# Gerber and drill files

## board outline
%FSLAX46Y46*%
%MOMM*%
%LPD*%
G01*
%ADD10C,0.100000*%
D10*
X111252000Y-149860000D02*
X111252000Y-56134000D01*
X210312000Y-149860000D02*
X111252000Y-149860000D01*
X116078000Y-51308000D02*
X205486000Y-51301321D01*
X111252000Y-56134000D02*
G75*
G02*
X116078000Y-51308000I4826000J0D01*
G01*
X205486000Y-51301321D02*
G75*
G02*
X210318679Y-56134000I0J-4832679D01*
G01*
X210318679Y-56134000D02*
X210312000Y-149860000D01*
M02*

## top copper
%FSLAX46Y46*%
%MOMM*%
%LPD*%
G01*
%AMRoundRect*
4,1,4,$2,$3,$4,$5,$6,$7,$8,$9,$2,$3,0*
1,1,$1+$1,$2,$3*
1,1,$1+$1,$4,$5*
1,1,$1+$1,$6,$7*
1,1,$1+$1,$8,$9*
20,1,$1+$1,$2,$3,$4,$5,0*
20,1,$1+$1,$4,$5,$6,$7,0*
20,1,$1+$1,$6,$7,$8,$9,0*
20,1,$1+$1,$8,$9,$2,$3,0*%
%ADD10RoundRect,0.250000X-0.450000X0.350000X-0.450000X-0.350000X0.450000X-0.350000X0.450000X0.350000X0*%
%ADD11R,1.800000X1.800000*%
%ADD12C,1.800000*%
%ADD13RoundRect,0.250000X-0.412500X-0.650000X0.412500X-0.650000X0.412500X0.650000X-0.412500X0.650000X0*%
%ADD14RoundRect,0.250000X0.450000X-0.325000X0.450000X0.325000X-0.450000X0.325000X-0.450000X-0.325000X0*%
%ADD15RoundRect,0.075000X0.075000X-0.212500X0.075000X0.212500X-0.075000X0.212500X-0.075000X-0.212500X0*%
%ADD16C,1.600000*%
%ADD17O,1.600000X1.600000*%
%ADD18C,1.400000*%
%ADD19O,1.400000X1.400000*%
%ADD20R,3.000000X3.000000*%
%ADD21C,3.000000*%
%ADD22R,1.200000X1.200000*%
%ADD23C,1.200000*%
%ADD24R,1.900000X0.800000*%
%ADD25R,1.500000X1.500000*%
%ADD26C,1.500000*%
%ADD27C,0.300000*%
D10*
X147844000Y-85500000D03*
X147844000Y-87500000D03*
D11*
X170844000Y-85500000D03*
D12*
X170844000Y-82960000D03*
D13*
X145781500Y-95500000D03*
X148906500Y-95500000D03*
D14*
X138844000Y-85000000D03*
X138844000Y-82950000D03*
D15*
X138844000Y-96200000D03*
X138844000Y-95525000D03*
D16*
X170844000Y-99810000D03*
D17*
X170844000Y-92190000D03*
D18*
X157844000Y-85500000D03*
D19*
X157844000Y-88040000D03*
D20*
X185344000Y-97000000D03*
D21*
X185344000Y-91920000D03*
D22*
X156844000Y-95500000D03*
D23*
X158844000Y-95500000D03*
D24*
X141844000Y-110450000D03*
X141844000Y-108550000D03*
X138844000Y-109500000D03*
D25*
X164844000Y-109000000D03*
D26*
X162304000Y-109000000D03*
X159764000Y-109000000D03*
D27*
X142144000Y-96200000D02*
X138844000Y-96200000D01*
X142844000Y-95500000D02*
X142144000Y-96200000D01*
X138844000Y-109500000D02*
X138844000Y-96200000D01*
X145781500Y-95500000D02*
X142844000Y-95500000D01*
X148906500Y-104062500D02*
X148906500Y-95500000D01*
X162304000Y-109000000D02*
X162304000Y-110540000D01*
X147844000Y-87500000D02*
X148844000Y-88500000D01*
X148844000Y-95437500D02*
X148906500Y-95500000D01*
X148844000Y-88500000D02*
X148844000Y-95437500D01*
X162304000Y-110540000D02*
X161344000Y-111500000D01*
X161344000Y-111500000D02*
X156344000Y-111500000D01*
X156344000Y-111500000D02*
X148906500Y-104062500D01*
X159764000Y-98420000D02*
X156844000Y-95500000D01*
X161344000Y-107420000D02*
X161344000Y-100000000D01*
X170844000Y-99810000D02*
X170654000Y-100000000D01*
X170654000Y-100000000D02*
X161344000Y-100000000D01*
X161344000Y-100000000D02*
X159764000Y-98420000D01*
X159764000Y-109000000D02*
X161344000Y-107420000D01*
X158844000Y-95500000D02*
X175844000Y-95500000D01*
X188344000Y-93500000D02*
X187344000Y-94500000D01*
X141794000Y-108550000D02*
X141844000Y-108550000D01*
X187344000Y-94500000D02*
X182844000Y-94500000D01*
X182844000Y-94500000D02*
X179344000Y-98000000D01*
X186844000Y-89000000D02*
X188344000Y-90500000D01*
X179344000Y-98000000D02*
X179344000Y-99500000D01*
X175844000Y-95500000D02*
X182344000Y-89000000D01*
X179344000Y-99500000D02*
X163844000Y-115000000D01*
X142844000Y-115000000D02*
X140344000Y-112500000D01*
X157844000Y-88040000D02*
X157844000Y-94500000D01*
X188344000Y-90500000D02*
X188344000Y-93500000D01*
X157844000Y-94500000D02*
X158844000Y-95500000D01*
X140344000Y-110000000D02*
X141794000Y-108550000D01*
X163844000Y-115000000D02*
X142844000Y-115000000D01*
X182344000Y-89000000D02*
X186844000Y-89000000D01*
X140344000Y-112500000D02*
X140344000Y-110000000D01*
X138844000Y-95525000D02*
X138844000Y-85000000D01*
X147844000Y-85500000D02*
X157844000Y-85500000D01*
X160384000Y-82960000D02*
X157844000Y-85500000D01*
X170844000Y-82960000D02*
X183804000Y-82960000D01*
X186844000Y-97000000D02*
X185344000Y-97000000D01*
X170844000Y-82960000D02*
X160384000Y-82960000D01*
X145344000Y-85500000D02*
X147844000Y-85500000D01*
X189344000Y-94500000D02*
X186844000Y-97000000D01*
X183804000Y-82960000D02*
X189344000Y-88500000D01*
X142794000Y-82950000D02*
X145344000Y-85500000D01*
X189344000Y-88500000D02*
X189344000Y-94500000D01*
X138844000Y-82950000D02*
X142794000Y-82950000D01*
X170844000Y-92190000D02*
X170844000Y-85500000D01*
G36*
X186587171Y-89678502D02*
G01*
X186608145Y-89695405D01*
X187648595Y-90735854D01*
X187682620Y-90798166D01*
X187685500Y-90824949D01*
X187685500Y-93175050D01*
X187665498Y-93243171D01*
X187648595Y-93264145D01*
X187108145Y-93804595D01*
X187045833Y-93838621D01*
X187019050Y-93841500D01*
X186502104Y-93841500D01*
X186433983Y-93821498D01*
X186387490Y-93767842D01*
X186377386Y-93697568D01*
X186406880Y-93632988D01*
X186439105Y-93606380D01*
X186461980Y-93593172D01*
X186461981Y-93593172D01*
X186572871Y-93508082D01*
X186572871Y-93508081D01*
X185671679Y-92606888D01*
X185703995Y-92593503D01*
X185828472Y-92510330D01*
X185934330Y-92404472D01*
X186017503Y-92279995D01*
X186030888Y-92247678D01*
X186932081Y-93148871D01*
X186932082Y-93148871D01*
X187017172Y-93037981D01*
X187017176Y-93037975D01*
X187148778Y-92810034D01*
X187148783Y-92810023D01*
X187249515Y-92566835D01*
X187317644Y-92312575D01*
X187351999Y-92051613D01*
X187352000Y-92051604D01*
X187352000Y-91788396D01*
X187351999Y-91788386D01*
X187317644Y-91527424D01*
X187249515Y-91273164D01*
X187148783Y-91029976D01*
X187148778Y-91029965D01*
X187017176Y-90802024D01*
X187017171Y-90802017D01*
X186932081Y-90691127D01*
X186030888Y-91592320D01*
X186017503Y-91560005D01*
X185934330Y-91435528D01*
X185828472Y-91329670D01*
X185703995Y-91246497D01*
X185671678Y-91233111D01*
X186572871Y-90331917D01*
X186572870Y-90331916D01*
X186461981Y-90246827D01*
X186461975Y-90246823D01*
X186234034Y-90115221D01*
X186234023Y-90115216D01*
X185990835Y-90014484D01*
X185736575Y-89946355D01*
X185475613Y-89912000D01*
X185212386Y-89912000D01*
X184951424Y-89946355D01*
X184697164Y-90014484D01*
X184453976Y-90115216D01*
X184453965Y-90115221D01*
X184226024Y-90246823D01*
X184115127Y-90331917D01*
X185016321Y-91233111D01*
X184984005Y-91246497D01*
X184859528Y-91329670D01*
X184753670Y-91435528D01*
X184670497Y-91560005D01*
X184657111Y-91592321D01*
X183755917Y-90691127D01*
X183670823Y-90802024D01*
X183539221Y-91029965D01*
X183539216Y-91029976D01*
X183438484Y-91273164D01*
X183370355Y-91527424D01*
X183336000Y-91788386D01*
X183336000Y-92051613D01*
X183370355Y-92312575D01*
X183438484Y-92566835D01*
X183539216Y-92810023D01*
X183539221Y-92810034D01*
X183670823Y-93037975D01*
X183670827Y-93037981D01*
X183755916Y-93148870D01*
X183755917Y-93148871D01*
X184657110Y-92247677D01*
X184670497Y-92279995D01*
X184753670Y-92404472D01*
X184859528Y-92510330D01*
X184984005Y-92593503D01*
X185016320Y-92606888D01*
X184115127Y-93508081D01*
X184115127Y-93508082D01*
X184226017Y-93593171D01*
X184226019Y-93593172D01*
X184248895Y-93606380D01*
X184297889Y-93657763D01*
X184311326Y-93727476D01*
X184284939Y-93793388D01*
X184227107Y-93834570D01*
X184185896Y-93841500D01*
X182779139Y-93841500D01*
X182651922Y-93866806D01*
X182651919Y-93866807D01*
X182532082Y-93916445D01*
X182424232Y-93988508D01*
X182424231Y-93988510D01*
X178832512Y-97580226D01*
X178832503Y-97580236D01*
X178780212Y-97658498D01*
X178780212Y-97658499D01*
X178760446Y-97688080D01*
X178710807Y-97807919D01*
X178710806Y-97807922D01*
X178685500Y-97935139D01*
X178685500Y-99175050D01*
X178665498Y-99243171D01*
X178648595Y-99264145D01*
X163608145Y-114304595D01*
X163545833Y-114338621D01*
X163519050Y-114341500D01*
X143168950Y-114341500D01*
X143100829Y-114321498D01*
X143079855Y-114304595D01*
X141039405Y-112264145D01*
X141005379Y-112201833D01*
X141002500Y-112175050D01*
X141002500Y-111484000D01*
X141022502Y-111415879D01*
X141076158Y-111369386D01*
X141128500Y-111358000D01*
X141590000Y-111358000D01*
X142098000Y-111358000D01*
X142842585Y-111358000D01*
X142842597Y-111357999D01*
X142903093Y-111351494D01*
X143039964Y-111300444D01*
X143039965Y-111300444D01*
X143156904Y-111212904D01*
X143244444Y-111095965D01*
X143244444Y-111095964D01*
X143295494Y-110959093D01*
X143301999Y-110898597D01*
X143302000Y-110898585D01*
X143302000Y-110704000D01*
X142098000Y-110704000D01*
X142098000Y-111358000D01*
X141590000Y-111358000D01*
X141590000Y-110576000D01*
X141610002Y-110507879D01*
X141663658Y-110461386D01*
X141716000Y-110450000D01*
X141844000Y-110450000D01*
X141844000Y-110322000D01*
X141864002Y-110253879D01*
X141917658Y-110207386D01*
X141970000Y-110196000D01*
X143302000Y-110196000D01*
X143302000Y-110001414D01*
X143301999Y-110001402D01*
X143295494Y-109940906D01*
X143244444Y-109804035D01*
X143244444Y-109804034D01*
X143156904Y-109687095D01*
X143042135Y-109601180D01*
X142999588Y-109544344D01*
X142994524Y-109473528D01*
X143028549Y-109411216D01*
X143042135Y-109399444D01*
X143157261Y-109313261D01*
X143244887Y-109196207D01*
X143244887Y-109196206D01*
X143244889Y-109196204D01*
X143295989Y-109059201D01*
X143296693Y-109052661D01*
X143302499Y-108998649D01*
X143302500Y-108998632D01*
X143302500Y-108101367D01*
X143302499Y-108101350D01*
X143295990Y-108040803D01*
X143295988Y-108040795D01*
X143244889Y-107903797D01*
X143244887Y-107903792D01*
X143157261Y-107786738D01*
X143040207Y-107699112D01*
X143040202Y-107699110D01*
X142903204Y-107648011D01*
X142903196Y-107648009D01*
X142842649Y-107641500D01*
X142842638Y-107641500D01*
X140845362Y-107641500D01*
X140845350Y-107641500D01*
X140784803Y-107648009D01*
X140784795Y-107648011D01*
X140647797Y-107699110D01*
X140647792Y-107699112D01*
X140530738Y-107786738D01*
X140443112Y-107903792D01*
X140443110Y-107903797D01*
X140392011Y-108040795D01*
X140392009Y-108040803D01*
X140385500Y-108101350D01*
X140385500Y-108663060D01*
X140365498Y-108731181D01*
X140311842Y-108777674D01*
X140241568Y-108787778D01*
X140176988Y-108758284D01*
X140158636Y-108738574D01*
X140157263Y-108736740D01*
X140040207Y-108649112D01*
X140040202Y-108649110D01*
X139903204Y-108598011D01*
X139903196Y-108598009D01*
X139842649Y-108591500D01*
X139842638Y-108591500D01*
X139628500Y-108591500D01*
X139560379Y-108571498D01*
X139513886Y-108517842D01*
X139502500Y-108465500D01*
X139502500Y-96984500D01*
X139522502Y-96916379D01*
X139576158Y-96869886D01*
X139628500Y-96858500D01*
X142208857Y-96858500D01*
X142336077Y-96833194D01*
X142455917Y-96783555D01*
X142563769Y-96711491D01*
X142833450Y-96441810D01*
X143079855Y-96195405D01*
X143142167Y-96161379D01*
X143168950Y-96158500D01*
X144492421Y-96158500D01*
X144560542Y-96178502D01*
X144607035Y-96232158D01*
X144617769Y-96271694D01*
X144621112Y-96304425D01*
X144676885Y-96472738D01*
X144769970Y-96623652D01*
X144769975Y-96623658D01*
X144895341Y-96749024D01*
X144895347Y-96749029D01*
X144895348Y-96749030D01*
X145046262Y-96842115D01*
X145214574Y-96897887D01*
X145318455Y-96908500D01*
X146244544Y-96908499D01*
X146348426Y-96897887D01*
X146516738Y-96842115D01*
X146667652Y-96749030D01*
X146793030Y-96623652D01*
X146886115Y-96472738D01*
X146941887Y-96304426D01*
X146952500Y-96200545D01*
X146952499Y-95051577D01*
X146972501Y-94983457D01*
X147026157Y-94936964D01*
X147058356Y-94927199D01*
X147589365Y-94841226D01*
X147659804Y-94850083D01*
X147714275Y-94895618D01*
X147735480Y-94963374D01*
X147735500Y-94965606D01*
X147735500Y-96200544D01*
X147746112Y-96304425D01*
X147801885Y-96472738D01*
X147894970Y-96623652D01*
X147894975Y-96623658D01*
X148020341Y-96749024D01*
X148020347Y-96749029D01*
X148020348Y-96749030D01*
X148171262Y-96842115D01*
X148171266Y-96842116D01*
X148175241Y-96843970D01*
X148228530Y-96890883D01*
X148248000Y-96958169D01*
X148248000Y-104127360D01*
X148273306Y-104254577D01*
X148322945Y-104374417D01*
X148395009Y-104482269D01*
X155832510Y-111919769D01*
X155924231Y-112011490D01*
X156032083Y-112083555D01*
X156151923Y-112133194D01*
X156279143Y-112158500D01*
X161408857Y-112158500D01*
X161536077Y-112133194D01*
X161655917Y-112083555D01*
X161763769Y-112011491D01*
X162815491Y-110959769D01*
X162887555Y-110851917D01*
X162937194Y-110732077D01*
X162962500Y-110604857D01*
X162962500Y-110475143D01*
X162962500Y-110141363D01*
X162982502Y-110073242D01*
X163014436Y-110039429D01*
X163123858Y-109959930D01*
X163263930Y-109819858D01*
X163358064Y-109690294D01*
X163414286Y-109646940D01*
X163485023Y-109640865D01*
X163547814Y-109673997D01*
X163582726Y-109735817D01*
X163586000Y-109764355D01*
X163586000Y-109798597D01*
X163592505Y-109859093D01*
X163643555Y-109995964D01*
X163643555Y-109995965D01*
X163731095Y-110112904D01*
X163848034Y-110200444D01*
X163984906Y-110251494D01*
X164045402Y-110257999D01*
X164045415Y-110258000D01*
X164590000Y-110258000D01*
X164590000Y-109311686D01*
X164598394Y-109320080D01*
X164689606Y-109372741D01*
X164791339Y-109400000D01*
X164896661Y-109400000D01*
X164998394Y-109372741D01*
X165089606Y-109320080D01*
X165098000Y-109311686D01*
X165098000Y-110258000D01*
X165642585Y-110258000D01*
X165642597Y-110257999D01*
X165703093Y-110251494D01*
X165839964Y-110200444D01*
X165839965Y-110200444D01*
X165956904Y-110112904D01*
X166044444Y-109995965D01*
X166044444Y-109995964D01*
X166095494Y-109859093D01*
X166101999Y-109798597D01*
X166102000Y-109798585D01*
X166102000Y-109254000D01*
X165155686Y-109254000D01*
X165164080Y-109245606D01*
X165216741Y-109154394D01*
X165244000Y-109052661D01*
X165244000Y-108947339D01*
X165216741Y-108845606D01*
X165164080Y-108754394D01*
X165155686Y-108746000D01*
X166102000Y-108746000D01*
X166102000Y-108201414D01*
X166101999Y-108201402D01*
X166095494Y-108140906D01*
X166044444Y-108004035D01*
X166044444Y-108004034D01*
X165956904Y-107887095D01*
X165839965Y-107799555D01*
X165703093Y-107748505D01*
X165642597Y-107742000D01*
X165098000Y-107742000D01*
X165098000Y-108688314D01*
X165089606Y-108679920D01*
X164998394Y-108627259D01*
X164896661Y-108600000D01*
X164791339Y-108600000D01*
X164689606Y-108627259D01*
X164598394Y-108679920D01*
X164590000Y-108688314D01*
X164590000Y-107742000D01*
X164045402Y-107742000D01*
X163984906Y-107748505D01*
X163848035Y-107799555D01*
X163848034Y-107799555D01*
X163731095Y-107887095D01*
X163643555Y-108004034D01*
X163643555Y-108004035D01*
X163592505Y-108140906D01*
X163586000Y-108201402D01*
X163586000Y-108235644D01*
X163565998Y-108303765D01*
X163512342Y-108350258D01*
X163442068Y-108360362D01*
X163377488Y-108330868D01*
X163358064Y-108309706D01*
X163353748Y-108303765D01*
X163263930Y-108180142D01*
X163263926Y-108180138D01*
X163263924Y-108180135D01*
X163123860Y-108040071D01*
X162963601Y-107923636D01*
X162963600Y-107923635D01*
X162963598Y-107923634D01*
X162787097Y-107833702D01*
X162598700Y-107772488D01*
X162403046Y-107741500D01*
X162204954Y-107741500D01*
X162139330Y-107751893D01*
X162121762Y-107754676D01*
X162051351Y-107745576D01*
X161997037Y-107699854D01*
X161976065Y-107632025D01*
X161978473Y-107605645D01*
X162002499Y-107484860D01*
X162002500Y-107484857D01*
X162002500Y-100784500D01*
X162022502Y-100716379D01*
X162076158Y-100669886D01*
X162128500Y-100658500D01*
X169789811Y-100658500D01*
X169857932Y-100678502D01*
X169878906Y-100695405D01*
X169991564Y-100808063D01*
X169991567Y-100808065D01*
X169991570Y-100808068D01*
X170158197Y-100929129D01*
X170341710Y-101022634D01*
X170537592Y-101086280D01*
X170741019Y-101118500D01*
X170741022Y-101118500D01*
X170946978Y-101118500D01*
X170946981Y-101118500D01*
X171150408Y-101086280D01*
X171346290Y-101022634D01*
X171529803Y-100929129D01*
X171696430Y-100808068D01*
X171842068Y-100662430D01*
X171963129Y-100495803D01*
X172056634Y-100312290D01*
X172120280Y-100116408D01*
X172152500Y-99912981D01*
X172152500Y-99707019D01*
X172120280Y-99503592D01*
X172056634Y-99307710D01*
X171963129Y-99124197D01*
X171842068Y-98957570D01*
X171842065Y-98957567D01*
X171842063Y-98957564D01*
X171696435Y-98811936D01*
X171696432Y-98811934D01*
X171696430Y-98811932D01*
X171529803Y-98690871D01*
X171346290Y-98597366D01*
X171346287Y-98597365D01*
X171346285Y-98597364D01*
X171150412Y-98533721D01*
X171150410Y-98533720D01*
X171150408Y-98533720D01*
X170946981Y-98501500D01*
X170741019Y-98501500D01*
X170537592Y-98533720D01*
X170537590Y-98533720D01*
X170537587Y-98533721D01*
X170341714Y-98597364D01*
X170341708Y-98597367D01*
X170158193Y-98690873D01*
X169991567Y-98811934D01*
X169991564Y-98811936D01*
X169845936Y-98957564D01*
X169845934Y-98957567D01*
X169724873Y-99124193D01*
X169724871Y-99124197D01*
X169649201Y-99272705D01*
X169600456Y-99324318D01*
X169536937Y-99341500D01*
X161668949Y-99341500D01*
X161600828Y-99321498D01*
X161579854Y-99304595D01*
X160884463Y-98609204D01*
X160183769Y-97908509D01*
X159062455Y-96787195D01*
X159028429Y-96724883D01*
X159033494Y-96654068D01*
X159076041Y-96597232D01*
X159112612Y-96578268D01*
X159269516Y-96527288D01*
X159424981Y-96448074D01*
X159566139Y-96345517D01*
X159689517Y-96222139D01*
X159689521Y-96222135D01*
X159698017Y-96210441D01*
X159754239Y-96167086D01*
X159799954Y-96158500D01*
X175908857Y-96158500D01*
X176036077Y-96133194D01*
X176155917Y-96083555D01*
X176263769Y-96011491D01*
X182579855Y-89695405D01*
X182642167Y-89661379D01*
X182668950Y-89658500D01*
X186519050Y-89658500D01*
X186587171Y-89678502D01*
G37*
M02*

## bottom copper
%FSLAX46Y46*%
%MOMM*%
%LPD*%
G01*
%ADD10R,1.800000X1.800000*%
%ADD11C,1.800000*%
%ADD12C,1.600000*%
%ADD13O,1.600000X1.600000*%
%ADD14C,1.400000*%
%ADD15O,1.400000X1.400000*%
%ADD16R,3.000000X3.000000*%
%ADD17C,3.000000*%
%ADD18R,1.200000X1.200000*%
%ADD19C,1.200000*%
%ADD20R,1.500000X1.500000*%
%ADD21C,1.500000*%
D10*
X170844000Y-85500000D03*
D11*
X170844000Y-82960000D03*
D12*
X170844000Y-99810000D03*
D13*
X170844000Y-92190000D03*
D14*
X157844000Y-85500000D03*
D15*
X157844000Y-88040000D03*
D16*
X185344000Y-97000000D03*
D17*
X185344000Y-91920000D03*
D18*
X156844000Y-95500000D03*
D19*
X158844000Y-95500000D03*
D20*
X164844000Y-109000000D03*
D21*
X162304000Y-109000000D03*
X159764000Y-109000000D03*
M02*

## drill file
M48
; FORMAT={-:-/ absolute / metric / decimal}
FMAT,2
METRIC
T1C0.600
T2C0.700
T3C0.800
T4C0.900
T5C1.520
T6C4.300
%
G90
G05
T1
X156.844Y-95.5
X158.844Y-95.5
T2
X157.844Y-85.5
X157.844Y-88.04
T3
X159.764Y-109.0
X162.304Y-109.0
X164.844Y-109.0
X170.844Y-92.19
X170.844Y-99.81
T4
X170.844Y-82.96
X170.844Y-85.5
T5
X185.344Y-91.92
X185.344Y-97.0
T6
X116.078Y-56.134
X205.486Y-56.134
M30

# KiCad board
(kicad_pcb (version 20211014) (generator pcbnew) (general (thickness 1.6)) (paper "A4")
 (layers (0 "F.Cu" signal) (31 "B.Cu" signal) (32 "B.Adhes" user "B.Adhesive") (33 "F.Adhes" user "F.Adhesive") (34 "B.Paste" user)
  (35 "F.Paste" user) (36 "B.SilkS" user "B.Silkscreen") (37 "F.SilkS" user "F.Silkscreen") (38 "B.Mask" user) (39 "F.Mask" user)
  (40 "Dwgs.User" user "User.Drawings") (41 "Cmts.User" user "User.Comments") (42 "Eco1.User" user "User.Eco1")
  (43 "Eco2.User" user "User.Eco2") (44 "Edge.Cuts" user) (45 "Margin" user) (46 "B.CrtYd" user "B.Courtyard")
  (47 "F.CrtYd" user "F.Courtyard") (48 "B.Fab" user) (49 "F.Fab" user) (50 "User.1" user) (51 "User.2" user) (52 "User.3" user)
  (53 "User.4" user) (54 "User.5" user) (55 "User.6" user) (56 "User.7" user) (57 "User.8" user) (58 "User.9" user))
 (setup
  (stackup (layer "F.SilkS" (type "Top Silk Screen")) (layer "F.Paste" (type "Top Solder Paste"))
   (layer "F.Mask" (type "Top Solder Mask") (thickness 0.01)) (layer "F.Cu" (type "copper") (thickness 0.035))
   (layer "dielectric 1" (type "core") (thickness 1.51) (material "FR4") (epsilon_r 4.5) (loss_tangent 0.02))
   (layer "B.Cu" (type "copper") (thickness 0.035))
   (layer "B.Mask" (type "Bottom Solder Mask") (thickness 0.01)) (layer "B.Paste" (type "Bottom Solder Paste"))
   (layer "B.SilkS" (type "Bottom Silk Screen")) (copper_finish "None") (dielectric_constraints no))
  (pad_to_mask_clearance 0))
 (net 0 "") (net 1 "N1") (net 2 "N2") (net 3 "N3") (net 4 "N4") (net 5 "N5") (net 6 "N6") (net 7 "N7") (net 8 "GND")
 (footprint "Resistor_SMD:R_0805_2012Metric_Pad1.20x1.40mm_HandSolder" (layer "F.Cu") (at 147.844 86.5 -90)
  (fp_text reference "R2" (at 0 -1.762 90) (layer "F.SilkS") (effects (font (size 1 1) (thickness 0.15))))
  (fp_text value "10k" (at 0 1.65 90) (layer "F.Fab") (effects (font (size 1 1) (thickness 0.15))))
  (pad "1" smd roundrect (at -1 0 270) (size 1.2 1.4) (layers "F.Cu" "F.Paste" "F.Mask") (roundrect_rratio 0.208333) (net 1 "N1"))
  (pad "2" smd roundrect (at 1 0 270) (size 1.2 1.4) (layers "F.Cu" "F.Paste" "F.Mask") (roundrect_rratio 0.208333) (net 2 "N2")))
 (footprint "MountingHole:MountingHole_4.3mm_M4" (layer "F.Cu") (at 205.486 56.134)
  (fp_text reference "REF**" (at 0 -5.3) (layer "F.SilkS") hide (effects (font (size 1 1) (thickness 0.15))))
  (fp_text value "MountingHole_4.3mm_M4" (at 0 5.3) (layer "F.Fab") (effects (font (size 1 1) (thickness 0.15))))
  (pad "" np_thru_hole circle (at 0 0) (size 4.3 4.3) (drill 4.3) (layers *.Cu *.Mask)))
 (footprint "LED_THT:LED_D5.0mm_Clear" (layer "F.Cu") (at 170.844 85.5 90)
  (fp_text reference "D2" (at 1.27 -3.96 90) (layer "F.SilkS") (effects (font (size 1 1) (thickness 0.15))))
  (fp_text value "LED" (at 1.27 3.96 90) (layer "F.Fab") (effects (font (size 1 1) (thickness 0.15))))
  (pad "1" thru_hole rect (at 0 0 90) (size 1.8 1.8) (drill 0.9) (layers *.Cu *.Mask) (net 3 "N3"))
  (pad "2" thru_hole circle (at 2.54 0 90) (size 1.8 1.8) (drill 0.9) (layers *.Cu *.Mask) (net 1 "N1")))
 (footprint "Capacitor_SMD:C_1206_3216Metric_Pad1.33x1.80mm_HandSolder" (layer "F.Cu") (at 147.344 95.5)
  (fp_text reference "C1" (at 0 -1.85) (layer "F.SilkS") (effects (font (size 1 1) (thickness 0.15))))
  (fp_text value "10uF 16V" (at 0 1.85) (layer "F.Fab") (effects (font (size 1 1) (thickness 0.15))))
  (pad "1" smd roundrect (at -1.5625 0) (size 1.325 1.8) (layers "F.Cu" "F.Paste" "F.Mask") (roundrect_rratio 0.188679) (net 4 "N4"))
  (pad "2" smd roundrect (at 1.5625 0) (size 1.325 1.8) (layers "F.Cu" "F.Paste" "F.Mask") (roundrect_rratio 0.188679) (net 2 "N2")))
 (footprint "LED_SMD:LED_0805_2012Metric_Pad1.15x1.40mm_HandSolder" (layer "F.Cu") (at 138.844 83.975 90)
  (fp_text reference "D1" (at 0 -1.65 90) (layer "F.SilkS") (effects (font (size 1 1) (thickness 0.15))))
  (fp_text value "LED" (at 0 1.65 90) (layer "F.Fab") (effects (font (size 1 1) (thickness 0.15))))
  (pad "1" smd roundrect (at -1.025 0 90) (size 1.15 1.4) (layers "F.Cu" "F.Paste" "F.Mask") (roundrect_rratio 0.217391) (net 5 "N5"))
  (pad "2" smd roundrect (at 1.025 0 90) (size 1.15 1.4) (layers "F.Cu" "F.Paste" "F.Mask") (roundrect_rratio 0.217391) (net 1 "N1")))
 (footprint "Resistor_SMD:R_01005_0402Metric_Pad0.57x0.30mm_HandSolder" (layer "F.Cu") (at 138.844 95.8625 90)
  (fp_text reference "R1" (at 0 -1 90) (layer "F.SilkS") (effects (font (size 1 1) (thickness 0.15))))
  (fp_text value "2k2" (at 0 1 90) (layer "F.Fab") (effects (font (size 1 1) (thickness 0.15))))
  (pad "" smd roundrect (at 0.3625 0 90) (size 0.41 0.27) (layers "F.Paste") (roundrect_rratio 0.25))
  (pad "" smd roundrect (at -0.3625 0 90) (size 0.41 0.27) (layers "F.Paste") (roundrect_rratio 0.25))
  (pad "1" smd roundrect (at -0.3375 0 90) (size 0.575 0.3) (layers "F.Cu" "F.Mask") (roundrect_rratio 0.25) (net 4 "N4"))
  (pad "2" smd roundrect (at 0.3375 0 90) (size 0.575 0.3) (layers "F.Cu" "F.Mask") (roundrect_rratio 0.25) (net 5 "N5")))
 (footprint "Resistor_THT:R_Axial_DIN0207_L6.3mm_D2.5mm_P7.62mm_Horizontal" (layer "F.Cu") (at 170.844 99.81 90)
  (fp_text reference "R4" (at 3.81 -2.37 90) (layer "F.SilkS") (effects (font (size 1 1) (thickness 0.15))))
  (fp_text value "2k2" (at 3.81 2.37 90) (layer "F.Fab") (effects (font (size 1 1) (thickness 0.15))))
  (pad "1" thru_hole circle (at 0 0 90) (size 1.6 1.6) (drill 0.8) (layers *.Cu *.Mask) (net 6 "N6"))
  (pad "2" thru_hole oval (at 7.62 0 90) (size 1.6 1.6) (drill 0.8) (layers *.Cu *.Mask) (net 3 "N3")))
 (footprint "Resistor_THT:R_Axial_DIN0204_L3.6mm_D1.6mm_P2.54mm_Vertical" (layer "F.Cu") (at 157.844 85.5 -90)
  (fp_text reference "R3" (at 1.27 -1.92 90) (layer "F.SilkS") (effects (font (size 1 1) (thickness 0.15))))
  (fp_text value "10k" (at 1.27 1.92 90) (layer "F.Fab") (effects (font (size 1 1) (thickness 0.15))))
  (pad "1" thru_hole circle (at 0 0 270) (size 1.4 1.4) (drill 0.7) (layers *.Cu *.Mask) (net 1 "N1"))
  (pad "2" thru_hole oval (at 2.54 0 270) (size 1.4 1.4) (drill 0.7) (layers *.Cu *.Mask) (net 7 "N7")))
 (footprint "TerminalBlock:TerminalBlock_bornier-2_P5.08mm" (layer "F.Cu") (at 185.344 97 90)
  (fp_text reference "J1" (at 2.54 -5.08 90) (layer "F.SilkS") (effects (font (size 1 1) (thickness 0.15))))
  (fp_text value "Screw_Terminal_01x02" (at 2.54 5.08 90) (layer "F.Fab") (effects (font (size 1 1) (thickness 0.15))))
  (pad "1" thru_hole rect (at 0 0 90) (size 3 3) (drill 1.52) (layers *.Cu *.Mask) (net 1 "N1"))
  (pad "2" thru_hole circle (at 5.08 0 90) (size 3 3) (drill 1.52) (layers *.Cu *.Mask) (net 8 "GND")))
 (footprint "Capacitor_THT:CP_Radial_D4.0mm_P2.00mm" (layer "F.Cu") (at 156.844 95.5)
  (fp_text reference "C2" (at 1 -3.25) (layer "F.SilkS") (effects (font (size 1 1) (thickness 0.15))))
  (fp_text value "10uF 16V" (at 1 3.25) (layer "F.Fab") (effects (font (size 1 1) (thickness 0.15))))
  (pad "1" thru_hole rect (at 0 0) (size 1.2 1.2) (drill 0.6) (layers *.Cu *.Mask) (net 6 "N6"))
  (pad "2" thru_hole circle (at 2 0) (size 1.2 1.2) (drill 0.6) (layers *.Cu *.Mask) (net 7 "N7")))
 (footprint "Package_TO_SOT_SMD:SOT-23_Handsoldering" (layer "F.Cu") (at 140.344 109.5 180)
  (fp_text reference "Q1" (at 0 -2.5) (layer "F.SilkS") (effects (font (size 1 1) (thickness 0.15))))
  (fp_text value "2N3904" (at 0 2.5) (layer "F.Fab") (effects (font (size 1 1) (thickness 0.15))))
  (pad "1" smd rect (at -1.5 -0.95 180) (size 1.9 0.8) (layers "F.Cu" "F.Paste" "F.Mask") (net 8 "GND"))
  (pad "2" smd rect (at -1.5 0.95 180) (size 1.9 0.8) (layers "F.Cu" "F.Paste" "F.Mask") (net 7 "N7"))
  (pad "3" smd rect (at 1.5 0 180) (size 1.9 0.8) (layers "F.Cu" "F.Paste" "F.Mask") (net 4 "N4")))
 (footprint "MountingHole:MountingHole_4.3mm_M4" (layer "F.Cu") (at 116.078 56.134)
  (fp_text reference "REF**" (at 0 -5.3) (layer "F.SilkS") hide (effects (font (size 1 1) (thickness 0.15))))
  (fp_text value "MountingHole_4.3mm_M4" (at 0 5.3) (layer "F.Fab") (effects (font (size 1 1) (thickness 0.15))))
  (pad "" np_thru_hole circle (at 0 0) (size 4.3 4.3) (drill 4.3) (layers *.Cu *.Mask)))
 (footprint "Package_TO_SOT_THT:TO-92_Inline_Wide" (layer "F.Cu") (at 164.844 109 180)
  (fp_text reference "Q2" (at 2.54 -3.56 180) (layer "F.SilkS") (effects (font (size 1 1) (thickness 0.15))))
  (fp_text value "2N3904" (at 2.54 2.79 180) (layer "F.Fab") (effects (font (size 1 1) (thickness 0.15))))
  (pad "1" thru_hole rect (at 0 0 180) (size 1.5 1.5) (drill 0.8) (layers *.Cu *.Mask) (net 8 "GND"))
  (pad "2" thru_hole circle (at 2.54 0 180) (size 1.5 1.5) (drill 0.8) (layers *.Cu *.Mask) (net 2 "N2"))
  (pad "3" thru_hole circle (at 5.08 0 180) (size 1.5 1.5) (drill 0.8) (layers *.Cu *.Mask) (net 6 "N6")))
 (gr_line (start 111.252 149.86) (end 111.252 56.134) (layer "Edge.Cuts") (width 0.1))
 (gr_line (start 210.312 149.86) (end 111.252 149.86) (layer "Edge.Cuts") (width 0.1))
 (gr_line (start 116.078 51.308) (end 205.486 51.301321) (layer "Edge.Cuts") (width 0.1))
 (gr_arc (start 111.252 56.134) (mid 112.665503 52.721503) (end 116.078 51.308) (layer "Edge.Cuts") (width 0.1))
 (gr_arc (start 205.486 51.301321) (mid 208.90322 52.71678) (end 210.318679 56.134) (layer "Edge.Cuts") (width 0.1))
 (gr_line (start 210.318679 56.134) (end 210.312 149.86) (layer "Edge.Cuts") (width 0.1))
 (segment (start 142.144 96.2) (end 138.844 96.2) (width 0.3) (layer "F.Cu") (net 4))
 (segment (start 142.844 95.5) (end 142.144 96.2) (width 0.3) (layer "F.Cu") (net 4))
 (segment (start 138.844 109.5) (end 138.844 96.2) (width 0.3) (layer "F.Cu") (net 4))
 (segment (start 145.7815 95.5) (end 142.844 95.5) (width 0.3) (layer "F.Cu") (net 4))
 (segment (start 148.9065 104.0625) (end 148.9065 95.5) (width 0.3) (layer "F.Cu") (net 2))
 (segment (start 162.304 109) (end 162.304 110.54) (width 0.3) (layer "F.Cu") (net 2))
 (segment (start 147.844 87.5) (end 148.844 88.5) (width 0.3) (layer "F.Cu") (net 2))
 (segment (start 148.844 95.4375) (end 148.9065 95.5) (width 0.3) (layer "F.Cu") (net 2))
 (segment (start 148.844 88.5) (end 148.844 95.4375) (width 0.3) (layer "F.Cu") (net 2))
 (segment (start 162.304 110.54) (end 161.344 111.5) (width 0.3) (layer "F.Cu") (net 2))
 (segment (start 161.344 111.5) (end 156.344 111.5) (width 0.3) (layer "F.Cu") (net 2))
 (segment (start 156.344 111.5) (end 148.9065 104.0625) (width 0.3) (layer "F.Cu") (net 2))
 (segment (start 159.764 98.42) (end 156.844 95.5) (width 0.3) (layer "F.Cu") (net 6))
 (segment (start 161.344 107.42) (end 161.344 100) (width 0.3) (layer "F.Cu") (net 6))
 (segment (start 170.844 99.81) (end 170.654 100) (width 0.3) (layer "F.Cu") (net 6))
 (segment (start 170.654 100) (end 161.344 100) (width 0.3) (layer "F.Cu") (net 6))
 (segment (start 161.344 100) (end 159.764 98.42) (width 0.3) (layer "F.Cu") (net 6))
 (segment (start 159.764 109) (end 161.344 107.42) (width 0.3) (layer "F.Cu") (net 6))
 (segment (start 158.844 95.5) (end 175.844 95.5) (width 0.3) (layer "F.Cu") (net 7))
 (segment (start 188.344 93.5) (end 187.344 94.5) (width 0.3) (layer "F.Cu") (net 7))
 (segment (start 141.794 108.55) (end 141.844 108.55) (width 0.3) (layer "F.Cu") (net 7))
 (segment (start 187.344 94.5) (end 182.844 94.5) (width 0.3) (layer "F.Cu") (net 7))
 (segment (start 182.844 94.5) (end 179.344 98) (width 0.3) (layer "F.Cu") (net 7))
 (segment (start 186.844 89) (end 188.344 90.5) (width 0.3) (layer "F.Cu") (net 7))
 (segment (start 179.344 98) (end 179.344 99.5) (width 0.3) (layer "F.Cu") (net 7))
 (segment (start 175.844 95.5) (end 182.344 89) (width 0.3) (layer "F.Cu") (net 7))
 (segment (start 179.344 99.5) (end 163.844 115) (width 0.3) (layer "F.Cu") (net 7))
 (segment (start 142.844 115) (end 140.344 112.5) (width 0.3) (layer "F.Cu") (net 7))
 (segment (start 157.844 88.04) (end 157.844 94.5) (width 0.3) (layer "F.Cu") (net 7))
 (segment (start 188.344 90.5) (end 188.344 93.5) (width 0.3) (layer "F.Cu") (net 7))
 (segment (start 157.844 94.5) (end 158.844 95.5) (width 0.3) (layer "F.Cu") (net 7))
 (segment (start 140.344 110) (end 141.794 108.55) (width 0.3) (layer "F.Cu") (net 7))
 (segment (start 163.844 115) (end 142.844 115) (width 0.3) (layer "F.Cu") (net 7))
 (segment (start 182.344 89) (end 186.844 89) (width 0.3) (layer "F.Cu") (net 7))
 (segment (start 140.344 112.5) (end 140.344 110) (width 0.3) (layer "F.Cu") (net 7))
 (segment (start 138.844 95.525) (end 138.844 85) (width 0.3) (layer "F.Cu") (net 5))
 (segment (start 147.844 85.5) (end 157.844 85.5) (width 0.3) (layer "F.Cu") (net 1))
 (segment (start 160.384 82.96) (end 157.844 85.5) (width 0.3) (layer "F.Cu") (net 1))
 (segment (start 170.844 82.96) (end 183.804 82.96) (width 0.3) (layer "F.Cu") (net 1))
 (segment (start 186.844 97) (end 185.344 97) (width 0.3) (layer "F.Cu") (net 1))
 (segment (start 170.844 82.96) (end 160.384 82.96) (width 0.3) (layer "F.Cu") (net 1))
 (segment (start 145.344 85.5) (end 147.844 85.5) (width 0.3) (layer "F.Cu") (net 1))
 (segment (start 189.344 94.5) (end 186.844 97) (width 0.3) (layer "F.Cu") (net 1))
 (segment (start 183.804 82.96) (end 189.344 88.5) (width 0.3) (layer "F.Cu") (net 1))
 (segment (start 142.794 82.95) (end 145.344 85.5) (width 0.3) (layer "F.Cu") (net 1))
 (segment (start 189.344 88.5) (end 189.344 94.5) (width 0.3) (layer "F.Cu") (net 1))
 (segment (start 138.844 82.95) (end 142.794 82.95) (width 0.3) (layer "F.Cu") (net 1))
 (segment (start 170.844 92.19) (end 170.844 85.5) (width 0.3) (layer "F.Cu") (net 3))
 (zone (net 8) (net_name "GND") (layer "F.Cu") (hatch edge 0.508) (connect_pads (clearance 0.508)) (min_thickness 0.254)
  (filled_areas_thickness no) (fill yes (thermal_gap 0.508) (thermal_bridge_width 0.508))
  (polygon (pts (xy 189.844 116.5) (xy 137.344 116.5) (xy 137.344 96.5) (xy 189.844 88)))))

